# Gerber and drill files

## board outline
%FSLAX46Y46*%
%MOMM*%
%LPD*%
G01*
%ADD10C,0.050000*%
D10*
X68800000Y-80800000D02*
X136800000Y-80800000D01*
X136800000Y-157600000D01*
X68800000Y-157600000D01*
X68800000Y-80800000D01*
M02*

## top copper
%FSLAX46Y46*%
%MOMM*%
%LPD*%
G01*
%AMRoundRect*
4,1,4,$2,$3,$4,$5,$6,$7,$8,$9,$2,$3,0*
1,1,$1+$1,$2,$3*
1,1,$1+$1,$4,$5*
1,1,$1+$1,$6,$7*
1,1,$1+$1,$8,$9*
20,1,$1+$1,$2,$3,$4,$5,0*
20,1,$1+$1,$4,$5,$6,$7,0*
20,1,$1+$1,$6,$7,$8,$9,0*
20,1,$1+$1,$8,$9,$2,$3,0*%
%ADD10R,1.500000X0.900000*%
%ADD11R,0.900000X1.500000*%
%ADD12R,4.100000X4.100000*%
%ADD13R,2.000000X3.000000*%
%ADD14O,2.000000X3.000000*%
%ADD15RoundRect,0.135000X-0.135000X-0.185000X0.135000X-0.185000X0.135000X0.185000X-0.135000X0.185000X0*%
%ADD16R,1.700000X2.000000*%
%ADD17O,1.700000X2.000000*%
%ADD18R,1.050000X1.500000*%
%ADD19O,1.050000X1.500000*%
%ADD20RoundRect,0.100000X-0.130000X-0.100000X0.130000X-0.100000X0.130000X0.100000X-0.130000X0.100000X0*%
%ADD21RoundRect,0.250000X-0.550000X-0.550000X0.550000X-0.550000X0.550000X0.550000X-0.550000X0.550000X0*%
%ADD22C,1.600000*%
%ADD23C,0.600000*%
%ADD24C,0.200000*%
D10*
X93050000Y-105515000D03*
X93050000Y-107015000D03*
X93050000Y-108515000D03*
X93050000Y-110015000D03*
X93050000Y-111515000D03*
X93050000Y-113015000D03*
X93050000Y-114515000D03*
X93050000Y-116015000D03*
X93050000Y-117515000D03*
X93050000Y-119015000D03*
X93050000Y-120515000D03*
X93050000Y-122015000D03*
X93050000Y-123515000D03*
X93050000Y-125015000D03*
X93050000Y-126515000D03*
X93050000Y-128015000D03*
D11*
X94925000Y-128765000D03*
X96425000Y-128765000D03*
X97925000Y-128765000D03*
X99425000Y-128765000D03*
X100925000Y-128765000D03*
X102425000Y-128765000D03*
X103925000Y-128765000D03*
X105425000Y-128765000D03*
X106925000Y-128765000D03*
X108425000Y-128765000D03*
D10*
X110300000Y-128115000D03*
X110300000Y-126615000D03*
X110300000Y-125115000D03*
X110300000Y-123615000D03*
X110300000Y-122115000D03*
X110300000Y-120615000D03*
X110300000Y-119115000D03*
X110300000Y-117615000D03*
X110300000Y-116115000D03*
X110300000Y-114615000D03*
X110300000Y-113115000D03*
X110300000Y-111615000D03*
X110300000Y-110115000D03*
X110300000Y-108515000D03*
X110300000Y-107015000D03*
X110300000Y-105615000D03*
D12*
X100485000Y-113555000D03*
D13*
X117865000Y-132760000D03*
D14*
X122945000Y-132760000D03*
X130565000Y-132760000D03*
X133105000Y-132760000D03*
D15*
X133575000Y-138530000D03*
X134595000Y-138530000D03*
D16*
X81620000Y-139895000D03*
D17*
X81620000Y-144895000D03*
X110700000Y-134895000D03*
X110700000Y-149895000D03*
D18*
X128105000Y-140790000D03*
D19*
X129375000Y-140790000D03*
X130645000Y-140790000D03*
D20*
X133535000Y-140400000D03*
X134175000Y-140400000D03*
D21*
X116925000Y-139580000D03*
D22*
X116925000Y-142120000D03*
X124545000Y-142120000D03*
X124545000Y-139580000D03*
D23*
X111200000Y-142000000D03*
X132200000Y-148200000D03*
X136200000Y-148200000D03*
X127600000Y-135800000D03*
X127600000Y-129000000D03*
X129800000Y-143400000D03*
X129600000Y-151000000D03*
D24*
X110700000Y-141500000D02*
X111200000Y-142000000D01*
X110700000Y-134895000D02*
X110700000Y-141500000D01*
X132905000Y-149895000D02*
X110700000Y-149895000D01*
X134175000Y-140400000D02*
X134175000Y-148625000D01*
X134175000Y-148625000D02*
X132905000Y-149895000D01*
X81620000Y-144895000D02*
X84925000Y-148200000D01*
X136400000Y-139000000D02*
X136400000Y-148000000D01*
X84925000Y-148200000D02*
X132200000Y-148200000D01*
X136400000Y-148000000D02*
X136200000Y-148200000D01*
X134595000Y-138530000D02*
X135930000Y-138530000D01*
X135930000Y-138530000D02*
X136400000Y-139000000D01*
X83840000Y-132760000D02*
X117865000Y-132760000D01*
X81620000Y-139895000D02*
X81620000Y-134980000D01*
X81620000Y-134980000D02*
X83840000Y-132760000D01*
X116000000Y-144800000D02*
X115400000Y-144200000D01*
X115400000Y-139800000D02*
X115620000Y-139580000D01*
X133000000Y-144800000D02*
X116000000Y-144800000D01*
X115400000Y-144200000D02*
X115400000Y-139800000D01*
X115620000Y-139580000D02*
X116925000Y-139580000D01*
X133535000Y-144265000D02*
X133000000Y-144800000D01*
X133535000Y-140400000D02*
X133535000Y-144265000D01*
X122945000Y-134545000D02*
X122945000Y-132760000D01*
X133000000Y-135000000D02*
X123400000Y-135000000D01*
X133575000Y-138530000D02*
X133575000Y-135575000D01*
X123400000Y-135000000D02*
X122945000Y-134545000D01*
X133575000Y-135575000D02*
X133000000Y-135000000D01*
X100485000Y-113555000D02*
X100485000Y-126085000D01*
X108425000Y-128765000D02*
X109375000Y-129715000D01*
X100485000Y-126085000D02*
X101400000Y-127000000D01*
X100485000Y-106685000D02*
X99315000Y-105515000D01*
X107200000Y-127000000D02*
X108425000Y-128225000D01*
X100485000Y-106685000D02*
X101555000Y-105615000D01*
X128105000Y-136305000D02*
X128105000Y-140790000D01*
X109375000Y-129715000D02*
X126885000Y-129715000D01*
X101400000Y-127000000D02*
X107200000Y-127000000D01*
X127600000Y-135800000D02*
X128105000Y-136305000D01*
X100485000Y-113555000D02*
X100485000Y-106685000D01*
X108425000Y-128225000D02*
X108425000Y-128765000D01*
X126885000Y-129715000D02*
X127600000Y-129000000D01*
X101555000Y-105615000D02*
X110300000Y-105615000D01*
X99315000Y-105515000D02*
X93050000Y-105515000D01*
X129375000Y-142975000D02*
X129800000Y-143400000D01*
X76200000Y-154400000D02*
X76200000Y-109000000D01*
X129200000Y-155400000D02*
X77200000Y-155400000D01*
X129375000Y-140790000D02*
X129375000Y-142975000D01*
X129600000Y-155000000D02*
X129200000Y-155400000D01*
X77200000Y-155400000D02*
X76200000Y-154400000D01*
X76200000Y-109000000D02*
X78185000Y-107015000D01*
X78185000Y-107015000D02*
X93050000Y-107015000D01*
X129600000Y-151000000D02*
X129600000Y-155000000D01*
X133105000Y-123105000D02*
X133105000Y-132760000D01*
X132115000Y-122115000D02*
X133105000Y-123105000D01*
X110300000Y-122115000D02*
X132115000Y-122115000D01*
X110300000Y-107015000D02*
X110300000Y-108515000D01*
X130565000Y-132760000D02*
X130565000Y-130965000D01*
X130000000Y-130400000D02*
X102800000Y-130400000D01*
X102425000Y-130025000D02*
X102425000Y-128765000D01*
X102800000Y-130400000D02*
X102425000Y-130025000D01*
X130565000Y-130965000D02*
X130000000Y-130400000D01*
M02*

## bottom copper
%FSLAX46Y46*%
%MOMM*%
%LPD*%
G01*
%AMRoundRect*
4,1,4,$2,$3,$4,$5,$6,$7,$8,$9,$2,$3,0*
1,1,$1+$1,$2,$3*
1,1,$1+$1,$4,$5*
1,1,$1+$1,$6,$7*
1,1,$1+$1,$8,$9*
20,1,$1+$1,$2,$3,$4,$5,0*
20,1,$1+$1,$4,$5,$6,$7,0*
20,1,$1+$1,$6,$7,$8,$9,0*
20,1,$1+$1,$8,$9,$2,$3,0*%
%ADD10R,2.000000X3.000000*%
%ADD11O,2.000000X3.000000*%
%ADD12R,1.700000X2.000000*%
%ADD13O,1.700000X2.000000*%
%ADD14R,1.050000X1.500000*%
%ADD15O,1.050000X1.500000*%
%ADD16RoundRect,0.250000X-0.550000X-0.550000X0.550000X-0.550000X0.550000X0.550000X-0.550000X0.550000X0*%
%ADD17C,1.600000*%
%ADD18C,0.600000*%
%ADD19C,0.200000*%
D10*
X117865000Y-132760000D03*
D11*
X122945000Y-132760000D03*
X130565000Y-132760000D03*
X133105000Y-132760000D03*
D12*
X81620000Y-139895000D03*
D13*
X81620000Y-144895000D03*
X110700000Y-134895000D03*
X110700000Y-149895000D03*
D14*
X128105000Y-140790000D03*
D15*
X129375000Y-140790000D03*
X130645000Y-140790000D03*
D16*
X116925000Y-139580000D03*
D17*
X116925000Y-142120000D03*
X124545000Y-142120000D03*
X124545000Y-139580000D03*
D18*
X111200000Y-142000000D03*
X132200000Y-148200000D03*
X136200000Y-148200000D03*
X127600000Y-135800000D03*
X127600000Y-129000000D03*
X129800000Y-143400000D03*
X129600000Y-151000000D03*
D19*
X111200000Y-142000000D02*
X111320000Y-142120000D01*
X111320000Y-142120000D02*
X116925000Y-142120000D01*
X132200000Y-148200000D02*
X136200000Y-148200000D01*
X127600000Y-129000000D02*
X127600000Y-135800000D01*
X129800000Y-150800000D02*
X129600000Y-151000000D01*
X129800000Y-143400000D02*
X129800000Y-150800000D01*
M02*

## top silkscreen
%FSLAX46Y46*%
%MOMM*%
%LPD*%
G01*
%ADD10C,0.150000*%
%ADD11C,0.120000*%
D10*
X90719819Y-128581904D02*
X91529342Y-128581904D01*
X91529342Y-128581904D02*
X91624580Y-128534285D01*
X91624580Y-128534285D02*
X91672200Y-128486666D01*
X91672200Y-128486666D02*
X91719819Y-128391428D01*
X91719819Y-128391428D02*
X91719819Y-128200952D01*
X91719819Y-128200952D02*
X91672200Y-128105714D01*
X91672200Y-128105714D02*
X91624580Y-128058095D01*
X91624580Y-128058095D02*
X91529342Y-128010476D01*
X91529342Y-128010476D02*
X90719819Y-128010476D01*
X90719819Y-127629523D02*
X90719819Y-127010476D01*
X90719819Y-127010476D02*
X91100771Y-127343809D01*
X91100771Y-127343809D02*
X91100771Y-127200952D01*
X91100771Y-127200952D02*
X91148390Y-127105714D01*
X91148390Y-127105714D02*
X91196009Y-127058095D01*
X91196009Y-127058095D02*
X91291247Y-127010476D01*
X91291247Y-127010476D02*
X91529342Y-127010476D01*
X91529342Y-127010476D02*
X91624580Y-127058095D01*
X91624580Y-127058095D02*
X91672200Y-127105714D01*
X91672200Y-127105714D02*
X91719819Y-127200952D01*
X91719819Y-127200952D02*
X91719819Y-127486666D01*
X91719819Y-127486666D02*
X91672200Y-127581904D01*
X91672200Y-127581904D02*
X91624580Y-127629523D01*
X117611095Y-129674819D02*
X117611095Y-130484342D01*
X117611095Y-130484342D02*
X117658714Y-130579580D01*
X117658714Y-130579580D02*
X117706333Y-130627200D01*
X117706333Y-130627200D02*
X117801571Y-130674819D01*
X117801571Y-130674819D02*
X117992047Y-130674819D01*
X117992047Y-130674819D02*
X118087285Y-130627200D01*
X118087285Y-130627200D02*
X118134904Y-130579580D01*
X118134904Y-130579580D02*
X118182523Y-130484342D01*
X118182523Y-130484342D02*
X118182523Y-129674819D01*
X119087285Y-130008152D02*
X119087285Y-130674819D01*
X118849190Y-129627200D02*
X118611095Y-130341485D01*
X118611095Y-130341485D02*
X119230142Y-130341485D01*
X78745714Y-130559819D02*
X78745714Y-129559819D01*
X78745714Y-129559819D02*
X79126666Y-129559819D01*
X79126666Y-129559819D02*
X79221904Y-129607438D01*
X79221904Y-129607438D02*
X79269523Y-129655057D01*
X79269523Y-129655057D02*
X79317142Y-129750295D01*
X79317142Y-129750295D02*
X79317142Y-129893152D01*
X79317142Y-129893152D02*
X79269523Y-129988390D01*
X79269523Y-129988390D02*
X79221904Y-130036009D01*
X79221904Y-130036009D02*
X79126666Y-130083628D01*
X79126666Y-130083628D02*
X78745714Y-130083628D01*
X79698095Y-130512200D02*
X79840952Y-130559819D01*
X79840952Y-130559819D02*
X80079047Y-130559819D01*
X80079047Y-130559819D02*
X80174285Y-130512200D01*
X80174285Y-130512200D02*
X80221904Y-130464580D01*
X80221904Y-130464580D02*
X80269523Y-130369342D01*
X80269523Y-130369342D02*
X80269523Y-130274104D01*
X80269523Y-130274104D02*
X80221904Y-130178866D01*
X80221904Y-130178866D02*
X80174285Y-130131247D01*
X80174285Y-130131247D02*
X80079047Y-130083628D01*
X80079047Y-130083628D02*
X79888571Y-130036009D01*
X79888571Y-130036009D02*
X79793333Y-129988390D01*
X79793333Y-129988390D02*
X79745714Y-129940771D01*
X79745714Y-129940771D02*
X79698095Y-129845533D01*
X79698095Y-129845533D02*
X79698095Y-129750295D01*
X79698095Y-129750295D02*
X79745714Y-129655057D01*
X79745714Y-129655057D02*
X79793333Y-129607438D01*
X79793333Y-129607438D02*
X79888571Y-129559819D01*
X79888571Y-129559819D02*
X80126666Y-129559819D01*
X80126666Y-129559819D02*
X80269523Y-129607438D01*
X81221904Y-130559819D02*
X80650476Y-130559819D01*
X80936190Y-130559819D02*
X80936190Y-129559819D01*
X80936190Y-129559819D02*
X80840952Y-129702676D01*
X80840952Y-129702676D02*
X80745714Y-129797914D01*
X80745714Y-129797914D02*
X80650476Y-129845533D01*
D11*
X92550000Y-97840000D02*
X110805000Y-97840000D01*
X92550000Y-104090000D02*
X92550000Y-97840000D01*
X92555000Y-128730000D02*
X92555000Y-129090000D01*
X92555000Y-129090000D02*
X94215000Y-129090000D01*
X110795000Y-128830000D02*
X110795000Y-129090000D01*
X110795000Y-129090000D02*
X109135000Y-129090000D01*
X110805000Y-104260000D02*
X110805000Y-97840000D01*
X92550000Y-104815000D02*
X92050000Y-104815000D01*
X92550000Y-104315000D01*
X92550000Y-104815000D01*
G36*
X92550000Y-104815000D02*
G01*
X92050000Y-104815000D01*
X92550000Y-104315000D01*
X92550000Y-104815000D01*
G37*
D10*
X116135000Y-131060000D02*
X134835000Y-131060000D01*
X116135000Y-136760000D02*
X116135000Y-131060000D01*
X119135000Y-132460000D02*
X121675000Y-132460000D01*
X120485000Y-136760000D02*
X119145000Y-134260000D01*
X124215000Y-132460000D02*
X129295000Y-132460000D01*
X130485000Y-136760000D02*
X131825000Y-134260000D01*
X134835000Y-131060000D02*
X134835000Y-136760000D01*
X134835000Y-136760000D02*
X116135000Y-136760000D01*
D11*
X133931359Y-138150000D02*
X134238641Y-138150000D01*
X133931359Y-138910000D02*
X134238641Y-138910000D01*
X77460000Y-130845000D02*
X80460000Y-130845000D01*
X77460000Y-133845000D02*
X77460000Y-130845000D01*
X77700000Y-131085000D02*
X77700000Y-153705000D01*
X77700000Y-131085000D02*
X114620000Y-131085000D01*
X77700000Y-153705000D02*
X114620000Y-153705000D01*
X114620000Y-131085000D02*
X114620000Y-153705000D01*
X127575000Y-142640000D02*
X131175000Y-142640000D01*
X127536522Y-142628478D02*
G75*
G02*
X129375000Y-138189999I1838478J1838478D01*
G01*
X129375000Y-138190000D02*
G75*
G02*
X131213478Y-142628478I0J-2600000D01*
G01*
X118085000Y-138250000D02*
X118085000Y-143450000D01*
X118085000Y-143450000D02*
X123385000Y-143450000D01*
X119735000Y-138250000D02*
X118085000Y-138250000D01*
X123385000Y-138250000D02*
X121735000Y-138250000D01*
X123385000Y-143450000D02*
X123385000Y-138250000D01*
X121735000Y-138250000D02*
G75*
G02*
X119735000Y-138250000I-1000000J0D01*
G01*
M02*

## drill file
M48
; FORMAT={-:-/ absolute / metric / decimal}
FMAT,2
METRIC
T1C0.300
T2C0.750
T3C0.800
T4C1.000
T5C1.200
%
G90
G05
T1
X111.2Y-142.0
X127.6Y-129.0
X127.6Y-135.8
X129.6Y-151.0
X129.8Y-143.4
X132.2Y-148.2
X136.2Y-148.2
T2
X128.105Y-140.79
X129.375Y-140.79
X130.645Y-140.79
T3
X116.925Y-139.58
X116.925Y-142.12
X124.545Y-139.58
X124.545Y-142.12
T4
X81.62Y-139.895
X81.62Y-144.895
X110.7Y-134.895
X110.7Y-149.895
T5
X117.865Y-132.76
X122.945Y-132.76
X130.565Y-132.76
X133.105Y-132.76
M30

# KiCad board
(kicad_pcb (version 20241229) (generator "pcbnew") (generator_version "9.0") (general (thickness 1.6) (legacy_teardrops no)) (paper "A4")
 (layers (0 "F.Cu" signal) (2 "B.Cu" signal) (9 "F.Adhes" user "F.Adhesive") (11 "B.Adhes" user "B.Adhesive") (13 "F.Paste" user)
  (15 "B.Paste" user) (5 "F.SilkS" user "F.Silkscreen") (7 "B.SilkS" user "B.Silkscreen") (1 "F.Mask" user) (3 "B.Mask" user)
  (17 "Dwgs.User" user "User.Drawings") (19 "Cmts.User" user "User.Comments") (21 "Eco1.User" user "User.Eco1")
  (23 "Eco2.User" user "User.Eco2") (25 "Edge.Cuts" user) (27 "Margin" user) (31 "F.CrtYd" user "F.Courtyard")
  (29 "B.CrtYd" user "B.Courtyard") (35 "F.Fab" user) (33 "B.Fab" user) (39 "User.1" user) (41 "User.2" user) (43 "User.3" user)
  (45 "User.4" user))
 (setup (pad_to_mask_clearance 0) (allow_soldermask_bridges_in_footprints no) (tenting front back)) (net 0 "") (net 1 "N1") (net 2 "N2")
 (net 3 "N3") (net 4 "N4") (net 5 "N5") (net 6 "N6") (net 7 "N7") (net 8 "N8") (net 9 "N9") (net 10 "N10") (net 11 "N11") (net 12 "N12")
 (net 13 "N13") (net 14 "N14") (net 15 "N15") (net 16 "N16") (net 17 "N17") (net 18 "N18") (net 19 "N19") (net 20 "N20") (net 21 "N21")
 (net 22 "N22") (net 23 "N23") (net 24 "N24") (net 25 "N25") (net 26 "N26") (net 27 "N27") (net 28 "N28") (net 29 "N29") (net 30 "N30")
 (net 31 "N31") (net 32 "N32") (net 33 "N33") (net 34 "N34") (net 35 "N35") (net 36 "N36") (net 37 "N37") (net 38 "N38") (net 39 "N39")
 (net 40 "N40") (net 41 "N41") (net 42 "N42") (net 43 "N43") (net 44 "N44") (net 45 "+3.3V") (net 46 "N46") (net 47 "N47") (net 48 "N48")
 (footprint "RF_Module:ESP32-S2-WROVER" (layer "F.Cu") (at 101.675 117.29)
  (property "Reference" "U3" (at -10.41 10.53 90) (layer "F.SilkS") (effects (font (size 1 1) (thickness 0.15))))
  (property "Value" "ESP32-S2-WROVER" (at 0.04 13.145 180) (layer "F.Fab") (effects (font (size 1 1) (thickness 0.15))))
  (fp_line (start -9.125 -19.45) (end 9.13 -19.45) (stroke (width 0.12) (type solid)) (layer "F.SilkS"))
  (fp_line (start -9.125 -13.2) (end -9.125 -19.45) (stroke (width 0.12) (type solid)) (layer "F.SilkS"))
  (fp_line (start -9.12 11.44) (end -9.12 11.8) (stroke (width 0.12) (type solid)) (layer "F.SilkS"))
  (fp_line (start -9.12 11.8) (end -7.46 11.8) (stroke (width 0.12) (type solid)) (layer "F.SilkS"))
  (fp_line (start 9.12 11.54) (end 9.12 11.8) (stroke (width 0.12) (type solid)) (layer "F.SilkS"))
  (fp_line (start 9.12 11.8) (end 7.46 11.8) (stroke (width 0.12) (type solid)) (layer "F.SilkS"))
  (fp_line (start 9.13 -13.03) (end 9.13 -19.45) (stroke (width 0.12) (type solid)) (layer "F.SilkS"))
  (fp_poly
   (pts (xy -9.125 -12.475) (xy -9.625 -12.475) (xy -9.125 -12.975) (xy -9.125 -12.475)) (stroke (width 0.12) (type solid)) (fill yes)
   (layer "F.SilkS"))
  (pad "" smd roundrect (at -2.52 -5.065) (size 1.07 1.07) (layers "F.Paste") (roundrect_rratio 0.233645))
  (pad "" smd roundrect (at -2.52 -3.735) (size 1.07 1.07) (layers "F.Paste") (roundrect_rratio 0.233645))
  (pad "" smd roundrect (at -2.52 -2.405) (size 1.07 1.07) (layers "F.Paste") (roundrect_rratio 0.233645))
  (pad "" smd roundrect (at -1.19 -5.065) (size 1.07 1.07) (layers "F.Paste") (roundrect_rratio 0.233645))
  (pad "" smd roundrect (at -1.19 -3.735) (size 1.07 1.07) (layers "F.Paste") (roundrect_rratio 0.233645))
  (pad "" smd roundrect (at -1.19 -2.405) (size 1.07 1.07) (layers "F.Paste") (roundrect_rratio 0.233645))
  (pad "" smd roundrect (at 0.14 -5.065) (size 1.07 1.07) (layers "F.Paste") (roundrect_rratio 0.233645))
  (pad "" smd roundrect (at 0.14 -3.735) (size 1.07 1.07) (layers "F.Paste") (roundrect_rratio 0.233645))
  (pad "" smd roundrect (at 0.14 -2.405) (size 1.07 1.07) (layers "F.Paste") (roundrect_rratio 0.233645))
  (pad "1" smd rect (at -8.625 -11.775) (size 1.5 0.9) (layers "F.Cu" "F.Mask" "F.Paste") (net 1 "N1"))
  (pad "2" smd rect (at -8.625 -10.275) (size 1.5 0.9) (layers "F.Cu" "F.Mask" "F.Paste") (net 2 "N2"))
  (pad "3" smd rect (at -8.625 -8.775) (size 1.5 0.9) (layers "F.Cu" "F.Mask" "F.Paste") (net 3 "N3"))
  (pad "4" smd rect (at -8.625 -7.275) (size 1.5 0.9) (layers "F.Cu" "F.Mask" "F.Paste") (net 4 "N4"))
  (pad "5" smd rect (at -8.625 -5.775) (size 1.5 0.9) (layers "F.Cu" "F.Mask" "F.Paste") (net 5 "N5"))
  (pad "6" smd rect (at -8.625 -4.275) (size 1.5 0.9) (layers "F.Cu" "F.Mask" "F.Paste") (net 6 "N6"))
  (pad "7" smd rect (at -8.625 -2.775) (size 1.5 0.9) (layers "F.Cu" "F.Mask" "F.Paste") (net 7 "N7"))
  (pad "8" smd rect (at -8.625 -1.275) (size 1.5 0.9) (layers "F.Cu" "F.Mask" "F.Paste") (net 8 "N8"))
  (pad "9" smd rect (at -8.625 0.225) (size 1.5 0.9) (layers "F.Cu" "F.Mask" "F.Paste") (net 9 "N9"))
  (pad "10" smd rect (at -8.625 1.725) (size 1.5 0.9) (layers "F.Cu" "F.Mask" "F.Paste") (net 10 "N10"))
  (pad "11" smd rect (at -8.625 3.225) (size 1.5 0.9) (layers "F.Cu" "F.Mask" "F.Paste") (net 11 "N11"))
  (pad "12" smd rect (at -8.625 4.725) (size 1.5 0.9) (layers "F.Cu" "F.Mask" "F.Paste") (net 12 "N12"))
  (pad "13" smd rect (at -8.625 6.225) (size 1.5 0.9) (layers "F.Cu" "F.Mask" "F.Paste") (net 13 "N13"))
  (pad "14" smd rect (at -8.625 7.725) (size 1.5 0.9) (layers "F.Cu" "F.Mask" "F.Paste") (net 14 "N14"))
  (pad "15" smd rect (at -8.625 9.225 180) (size 1.5 0.9) (layers "F.Cu" "F.Mask" "F.Paste") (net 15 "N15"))
  (pad "16" smd rect (at -8.625 10.725 180) (size 1.5 0.9) (layers "F.Cu" "F.Mask" "F.Paste") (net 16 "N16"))
  (pad "17" smd rect (at -6.75 11.475) (size 0.9 1.5) (layers "F.Cu" "F.Mask" "F.Paste") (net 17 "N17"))
  (pad "18" smd rect (at -5.25 11.475) (size 0.9 1.5) (layers "F.Cu" "F.Mask" "F.Paste") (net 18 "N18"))
  (pad "19" smd rect (at -3.75 11.475) (size 0.9 1.5) (layers "F.Cu" "F.Mask" "F.Paste") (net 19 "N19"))
  (pad "20" smd rect (at -2.25 11.475) (size 0.9 1.5) (layers "F.Cu" "F.Mask" "F.Paste") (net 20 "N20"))
  (pad "21" smd rect (at -0.75 11.475) (size 0.9 1.5) (layers "F.Cu" "F.Mask" "F.Paste") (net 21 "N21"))
  (pad "22" smd rect (at 0.75 11.475) (size 0.9 1.5) (layers "F.Cu" "F.Mask" "F.Paste") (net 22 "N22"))
  (pad "23" smd rect (at 2.25 11.475) (size 0.9 1.5) (layers "F.Cu" "F.Mask" "F.Paste") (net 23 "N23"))
  (pad "24" smd rect (at 3.75 11.475) (size 0.9 1.5) (layers "F.Cu" "F.Mask" "F.Paste") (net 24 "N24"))
  (pad "25" smd rect (at 5.25 11.475) (size 0.9 1.5) (layers "F.Cu" "F.Mask" "F.Paste") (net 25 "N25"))
  (pad "26" smd rect (at 6.75 11.475) (size 0.9 1.5) (layers "F.Cu" "F.Mask" "F.Paste") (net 1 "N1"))
  (pad "27" smd rect (at 8.625 10.825) (size 1.5 0.9) (layers "F.Cu" "F.Mask" "F.Paste") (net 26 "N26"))
  (pad "28" smd rect (at 8.625 9.325) (size 1.5 0.9) (layers "F.Cu" "F.Mask" "F.Paste") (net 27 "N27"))
  (pad "29" smd rect (at 8.625 7.825) (size 1.5 0.9) (layers "F.Cu" "F.Mask" "F.Paste") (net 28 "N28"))
  (pad "30" smd rect (at 8.625 6.325) (size 1.5 0.9) (layers "F.Cu" "F.Mask" "F.Paste") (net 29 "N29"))
  (pad "31" smd rect (at 8.625 4.825) (size 1.5 0.9) (layers "F.Cu" "F.Mask" "F.Paste") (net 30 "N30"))
  (pad "32" smd rect (at 8.625 3.325) (size 1.5 0.9) (layers "F.Cu" "F.Mask" "F.Paste") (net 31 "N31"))
  (pad "33" smd rect (at 8.625 1.825) (size 1.5 0.9) (layers "F.Cu" "F.Mask" "F.Paste") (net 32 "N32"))
  (pad "34" smd rect (at 8.625 0.325) (size 1.5 0.9) (layers "F.Cu" "F.Mask" "F.Paste") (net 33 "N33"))
  (pad "35" smd rect (at 8.625 -1.175) (size 1.5 0.9) (layers "F.Cu" "F.Mask" "F.Paste") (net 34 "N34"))
  (pad "36" smd rect (at 8.625 -2.675) (size 1.5 0.9) (layers "F.Cu" "F.Mask" "F.Paste") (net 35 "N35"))
  (pad "37" smd rect (at 8.625 -4.175) (size 1.5 0.9) (layers "F.Cu" "F.Mask" "F.Paste") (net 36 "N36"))
  (pad "38" smd rect (at 8.625 -5.675) (size 1.5 0.9) (layers "F.Cu" "F.Mask" "F.Paste") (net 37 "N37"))
  (pad "39" smd rect (at 8.625 -7.175) (size 1.5 0.9) (layers "F.Cu" "F.Mask" "F.Paste") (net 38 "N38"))
  (pad "40" smd rect (at 8.625 -8.775) (size 1.5 0.9) (layers "F.Cu" "F.Mask" "F.Paste") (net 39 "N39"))
  (pad "41" smd rect (at 8.625 -10.275) (size 1.5 0.9) (layers "F.Cu" "F.Mask" "F.Paste") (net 39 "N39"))
  (pad "42" smd rect (at 8.625 -11.675) (size 1.5 0.9) (layers "F.Cu" "F.Mask" "F.Paste") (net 1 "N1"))
  (pad "43" smd rect (at -1.19 -3.735) (size 4.1 4.1) (layers "F.Cu" "F.Mask") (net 1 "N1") (zone_connect 2))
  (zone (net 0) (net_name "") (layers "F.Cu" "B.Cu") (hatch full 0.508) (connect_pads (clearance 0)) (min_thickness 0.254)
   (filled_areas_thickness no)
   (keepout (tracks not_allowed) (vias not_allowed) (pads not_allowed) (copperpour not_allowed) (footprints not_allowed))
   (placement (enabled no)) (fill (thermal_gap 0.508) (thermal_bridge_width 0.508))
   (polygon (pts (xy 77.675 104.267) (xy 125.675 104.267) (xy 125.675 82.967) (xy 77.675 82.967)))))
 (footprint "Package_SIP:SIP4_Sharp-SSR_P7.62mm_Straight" (layer "F.Cu") (at 117.865 132.76)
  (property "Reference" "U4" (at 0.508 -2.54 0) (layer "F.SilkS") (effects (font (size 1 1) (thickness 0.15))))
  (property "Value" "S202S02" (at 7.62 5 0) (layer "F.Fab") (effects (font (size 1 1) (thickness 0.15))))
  (fp_line (start -1.73 -1.7) (end 16.97 -1.7) (stroke (width 0.15) (type solid)) (layer "F.SilkS"))
  (fp_line (start -1.73 4) (end -1.73 -1.7) (stroke (width 0.15) (type solid)) (layer "F.SilkS"))
  (fp_line (start 1.27 -0.3) (end 3.81 -0.3) (stroke (width 0.15) (type solid)) (layer "F.SilkS"))
  (fp_line (start 2.62 4) (end 1.28 1.5) (stroke (width 0.15) (type solid)) (layer "F.SilkS"))
  (fp_line (start 6.35 -0.3) (end 11.43 -0.3) (stroke (width 0.15) (type solid)) (layer "F.SilkS"))
  (fp_line (start 12.62 4) (end 13.96 1.5) (stroke (width 0.15) (type solid)) (layer "F.SilkS"))
  (fp_line (start 16.97 -1.7) (end 16.97 4) (stroke (width 0.15) (type solid)) (layer "F.SilkS"))
  (fp_line (start 16.97 4) (end -1.73 4) (stroke (width 0.15) (type solid)) (layer "F.SilkS"))
  (pad "1" thru_hole rect (at 0 0) (size 2 3) (drill 1.2) (layers "*.Cu" "*.Mask") (remove_unused_layers no) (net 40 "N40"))
  (pad "2" thru_hole oval (at 5.08 0) (size 2 3) (drill 1.2) (layers "*.Cu" "*.Mask") (remove_unused_layers no) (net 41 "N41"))
  (pad "3" thru_hole oval (at 12.7 0) (size 2 3) (drill 1.2) (layers "*.Cu" "*.Mask") (remove_unused_layers no) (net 22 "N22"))
  (pad "4" thru_hole oval (at 15.24 0) (size 2 3) (drill 1.2) (layers "*.Cu" "*.Mask") (remove_unused_layers no) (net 30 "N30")))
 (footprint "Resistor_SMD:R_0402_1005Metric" (layer "F.Cu") (at 134.085 138.53)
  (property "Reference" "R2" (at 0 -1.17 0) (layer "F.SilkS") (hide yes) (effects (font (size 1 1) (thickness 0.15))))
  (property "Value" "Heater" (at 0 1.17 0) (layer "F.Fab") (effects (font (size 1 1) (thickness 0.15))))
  (fp_line (start -0.153641 -0.38) (end 0.153641 -0.38) (stroke (width 0.12) (type solid)) (layer "F.SilkS"))
  (fp_line (start -0.153641 0.38) (end 0.153641 0.38) (stroke (width 0.12) (type solid)) (layer "F.SilkS"))
  (pad "1" smd roundrect (at -0.51 0) (size 0.54 0.64) (layers "F.Cu" "F.Mask" "F.Paste") (roundrect_rratio 0.25) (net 41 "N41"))
  (pad "2" smd roundrect (at 0.51 0) (size 0.54 0.64) (layers "F.Cu" "F.Mask" "F.Paste") (roundrect_rratio 0.25) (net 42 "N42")))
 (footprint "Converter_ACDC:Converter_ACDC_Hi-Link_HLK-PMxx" (layer "F.Cu") (at 81.62 139.895)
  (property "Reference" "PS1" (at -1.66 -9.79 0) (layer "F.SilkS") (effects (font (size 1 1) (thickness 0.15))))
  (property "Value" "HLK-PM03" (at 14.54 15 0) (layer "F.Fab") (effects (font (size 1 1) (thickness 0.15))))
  (fp_line (start -4.16 -9.05) (end -1.16 -9.05) (stroke (width 0.12) (type solid)) (layer "F.SilkS"))
  (fp_line (start -4.16 -6.05) (end -4.16 -9.05) (stroke (width 0.12) (type solid)) (layer "F.SilkS"))
  (fp_line (start -3.92 -8.81) (end -3.92 13.81) (stroke (width 0.12) (type solid)) (layer "F.SilkS"))
  (fp_line (start -3.92 -8.81) (end 33 -8.81) (stroke (width 0.12) (type solid)) (layer "F.SilkS"))
  (fp_line (start -3.92 13.81) (end 33 13.81) (stroke (width 0.12) (type solid)) (layer "F.SilkS"))
  (fp_line (start 33 -8.81) (end 33 13.81) (stroke (width 0.12) (type solid)) (layer "F.SilkS"))
  (pad "1" thru_hole rect (at 0 0) (size 1.7 2) (drill 1) (layers "*.Cu" "*.Mask") (remove_unused_layers no) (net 40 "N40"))
  (pad "2" thru_hole oval (at 0 5) (size 1.7 2) (drill 1) (layers "*.Cu" "*.Mask") (remove_unused_layers no) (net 42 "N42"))
  (pad "3" thru_hole oval (at 29.08 -5) (size 1.7 2) (drill 1) (layers "*.Cu" "*.Mask") (remove_unused_layers no) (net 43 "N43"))
  (pad "4" thru_hole oval (at 29.08 10) (size 1.7 2) (drill 1) (layers "*.Cu" "*.Mask") (remove_unused_layers no) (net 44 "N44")))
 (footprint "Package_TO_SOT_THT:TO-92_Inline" (layer "F.Cu") (at 128.105 140.79)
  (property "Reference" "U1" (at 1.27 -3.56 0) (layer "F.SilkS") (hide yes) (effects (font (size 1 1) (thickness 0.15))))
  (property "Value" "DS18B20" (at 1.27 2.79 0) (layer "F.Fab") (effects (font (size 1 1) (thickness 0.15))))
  (fp_line (start -0.53 1.85) (end 3.07 1.85) (stroke (width 0.12) (type solid)) (layer "F.SilkS"))
  (fp_arc (start -0.568478 1.838478) (mid -1.132087 -0.994977) (end 1.27 -2.6) (stroke (width 0.12) (type solid)) (layer "F.SilkS"))
  (fp_arc (start 1.27 -2.6) (mid 3.672087 -0.994977) (end 3.108478 1.838478) (stroke (width 0.12) (type solid)) (layer "F.SilkS"))
  (pad "1" thru_hole rect (at 0 0) (size 1.05 1.5) (drill 0.75) (layers "*.Cu" "*.Mask") (remove_unused_layers no) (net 1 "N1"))
  (pad "2" thru_hole oval (at 1.27 0) (size 1.05 1.5) (drill 0.75) (layers "*.Cu" "*.Mask") (remove_unused_layers no) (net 2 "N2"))
  (pad "3" thru_hole oval (at 2.54 0) (size 1.05 1.5) (drill 0.75) (layers "*.Cu" "*.Mask") (remove_unused_layers no) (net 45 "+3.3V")))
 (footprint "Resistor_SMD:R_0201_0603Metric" (layer "F.Cu") (at 133.855 140.4)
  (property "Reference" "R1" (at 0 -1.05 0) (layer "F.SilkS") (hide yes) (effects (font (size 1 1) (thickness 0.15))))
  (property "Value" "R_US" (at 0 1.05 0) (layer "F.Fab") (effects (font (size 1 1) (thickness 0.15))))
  (pad "" smd roundrect (at -0.345 0) (size 0.318 0.36) (layers "F.Paste") (roundrect_rratio 0.25))
  (pad "" smd roundrect (at 0.345 0) (size 0.318 0.36) (layers "F.Paste") (roundrect_rratio 0.25))
  (pad "1" smd roundrect (at -0.32 0) (size 0.46 0.4) (layers "F.Cu" "F.Mask") (roundrect_rratio 0.25) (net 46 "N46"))
  (pad "2" smd roundrect (at 0.32 0) (size 0.46 0.4) (layers "F.Cu" "F.Mask") (roundrect_rratio 0.25) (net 44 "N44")))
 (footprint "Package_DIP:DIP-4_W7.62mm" (layer "F.Cu") (at 116.925 139.58)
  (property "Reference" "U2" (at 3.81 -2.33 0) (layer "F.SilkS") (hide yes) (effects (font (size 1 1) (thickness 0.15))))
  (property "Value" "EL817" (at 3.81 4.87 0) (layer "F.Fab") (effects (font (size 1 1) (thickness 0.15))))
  (fp_line (start 1.16 -1.33) (end 1.16 3.87) (stroke (width 0.12) (type solid)) (layer "F.SilkS"))
  (fp_line (start 1.16 3.87) (end 6.46 3.87) (stroke (width 0.12) (type solid)) (layer "F.SilkS"))
  (fp_line (start 2.81 -1.33) (end 1.16 -1.33) (stroke (width 0.12) (type solid)) (layer "F.SilkS"))
  (fp_line (start 6.46 -1.33) (end 4.81 -1.33) (stroke (width 0.12) (type solid)) (layer "F.SilkS"))
  (fp_line (start 6.46 3.87) (end 6.46 -1.33) (stroke (width 0.12) (type solid)) (layer "F.SilkS"))
  (fp_arc (start 4.81 -1.33) (mid 3.81 -0.33) (end 2.81 -1.33) (stroke (width 0.12) (type solid)) (layer "F.SilkS"))
  (pad "1" thru_hole roundrect (at 0 0) (size 1.6 1.6) (drill 0.8) (layers "*.Cu" "*.Mask") (remove_unused_layers no)
   (roundrect_rratio 0.15625) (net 46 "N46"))
  (pad "2" thru_hole circle (at 0 2.54) (size 1.6 1.6) (drill 0.8) (layers "*.Cu" "*.Mask") (remove_unused_layers no) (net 43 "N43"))
  (pad "3" thru_hole circle (at 7.62 2.54) (size 1.6 1.6) (drill 0.8) (layers "*.Cu" "*.Mask") (remove_unused_layers no) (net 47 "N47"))
  (pad "4" thru_hole circle (at 7.62 0) (size 1.6 1.6) (drill 0.8) (layers "*.Cu" "*.Mask") (remove_unused_layers no) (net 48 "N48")))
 (gr_rect (start 68.8 80.8) (end 136.8 157.6) (stroke (width 0.05) (type default)) (fill no) (layer "Edge.Cuts"))
 (segment (start 110.7 141.5) (end 111.2 142) (width 0.2) (layer "F.Cu") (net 43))
 (segment (start 110.7 134.895) (end 110.7 141.5) (width 0.2) (layer "F.Cu") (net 43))
 (via (at 111.2 142) (size 0.6) (drill 0.3) (layers "F.Cu" "B.Cu") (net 43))
 (segment (start 111.2 142) (end 111.32 142.12) (width 0.2) (layer "B.Cu") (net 43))
 (segment (start 111.32 142.12) (end 116.925 142.12) (width 0.2) (layer "B.Cu") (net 43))
 (segment (start 132.905 149.895) (end 110.7 149.895) (width 0.2) (layer "F.Cu") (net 44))
 (segment (start 134.175 140.4) (end 134.175 148.625) (width 0.2) (layer "F.Cu") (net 44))
 (segment (start 134.175 148.625) (end 132.905 149.895) (width 0.2) (layer "F.Cu") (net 44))
 (segment (start 81.62 144.895) (end 84.925 148.2) (width 0.2) (layer "F.Cu") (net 42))
 (segment (start 136.4 139) (end 136.4 148) (width 0.2) (layer "F.Cu") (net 42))
 (segment (start 84.925 148.2) (end 132.2 148.2) (width 0.2) (layer "F.Cu") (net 42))
 (segment (start 136.4 148) (end 136.2 148.2) (width 0.2) (layer "F.Cu") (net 42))
 (segment (start 134.595 138.53) (end 135.93 138.53) (width 0.2) (layer "F.Cu") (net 42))
 (segment (start 135.93 138.53) (end 136.4 139) (width 0.2) (layer "F.Cu") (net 42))
 (via (at 132.2 148.2) (size 0.6) (drill 0.3) (layers "F.Cu" "B.Cu") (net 42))
 (via (at 136.2 148.2) (size 0.6) (drill 0.3) (layers "F.Cu" "B.Cu") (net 42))
 (segment (start 132.2 148.2) (end 136.2 148.2) (width 0.2) (layer "B.Cu") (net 42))
 (segment (start 83.84 132.76) (end 117.865 132.76) (width 0.2) (layer "F.Cu") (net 40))
 (segment (start 81.62 139.895) (end 81.62 134.98) (width 0.2) (layer "F.Cu") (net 40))
 (segment (start 81.62 134.98) (end 83.84 132.76) (width 0.2) (layer "F.Cu") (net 40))
 (segment (start 116 144.8) (end 115.4 144.2) (width 0.2) (layer "F.Cu") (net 46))
 (segment (start 115.4 139.8) (end 115.62 139.58) (width 0.2) (layer "F.Cu") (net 46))
 (segment (start 133 144.8) (end 116 144.8) (width 0.2) (layer "F.Cu") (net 46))
 (segment (start 115.4 144.2) (end 115.4 139.8) (width 0.2) (layer "F.Cu") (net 46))
 (segment (start 115.62 139.58) (end 116.925 139.58) (width 0.2) (layer "F.Cu") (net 46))
 (segment (start 133.535 144.265) (end 133 144.8) (width 0.2) (layer "F.Cu") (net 46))
 (segment (start 133.535 140.4) (end 133.535 144.265) (width 0.2) (layer "F.Cu") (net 46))
 (segment (start 122.945 134.545) (end 122.945 132.76) (width 0.2) (layer "F.Cu") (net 41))
 (segment (start 133 135) (end 123.4 135) (width 0.2) (layer "F.Cu") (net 41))
 (segment (start 133.575 138.53) (end 133.575 135.575) (width 0.2) (layer "F.Cu") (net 41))
 (segment (start 123.4 135) (end 122.945 134.545) (width 0.2) (layer "F.Cu") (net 41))
 (segment (start 133.575 135.575) (end 133 135) (width 0.2) (layer "F.Cu") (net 41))
 (segment (start 100.485 113.555) (end 100.485 126.085) (width 0.2) (layer "F.Cu") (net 1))
 (segment (start 108.425 128.765) (end 109.375 129.715) (width 0.2) (layer "F.Cu") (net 1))
 (segment (start 100.485 126.085) (end 101.4 127) (width 0.2) (layer "F.Cu") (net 1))
 (segment (start 100.485 106.685) (end 99.315 105.515) (width 0.2) (layer "F.Cu") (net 1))
 (segment (start 107.2 127) (end 108.425 128.225) (width 0.2) (layer "F.Cu") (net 1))
 (segment (start 100.485 106.685) (end 101.555 105.615) (width 0.2) (layer "F.Cu") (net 1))
 (segment (start 128.105 136.305) (end 128.105 140.79) (width 0.2) (layer "F.Cu") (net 1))
 (segment (start 109.375 129.715) (end 126.885 129.715) (width 0.2) (layer "F.Cu") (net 1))
 (segment (start 101.4 127) (end 107.2 127) (width 0.2) (layer "F.Cu") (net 1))
 (segment (start 127.6 135.8) (end 128.105 136.305) (width 0.2) (layer "F.Cu") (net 1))
 (segment (start 100.485 113.555) (end 100.485 106.685) (width 0.2) (layer "F.Cu") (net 1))
 (segment (start 108.425 128.225) (end 108.425 128.765) (width 0.2) (layer "F.Cu") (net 1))
 (segment (start 126.885 129.715) (end 127.6 129) (width 0.2) (layer "F.Cu") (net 1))
 (segment (start 101.555 105.615) (end 110.3 105.615) (width 0.2) (layer "F.Cu") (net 1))
 (segment (start 99.315 105.515) (end 93.05 105.515) (width 0.2) (layer "F.Cu") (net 1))
 (via (at 127.6 135.8) (size 0.6) (drill 0.3) (layers "F.Cu" "B.Cu") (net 1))
 (via (at 127.6 129) (size 0.6) (drill 0.3) (layers "F.Cu" "B.Cu") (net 1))
 (segment (start 127.6 129) (end 127.6 135.8) (width 0.2) (layer "B.Cu") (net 1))
 (segment (start 129.375 142.975) (end 129.8 143.4) (width 0.2) (layer "F.Cu") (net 2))
 (segment (start 76.2 154.4) (end 76.2 109) (width 0.2) (layer "F.Cu") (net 2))
 (segment (start 129.2 155.4) (end 77.2 155.4) (width 0.2) (layer "F.Cu") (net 2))
 (segment (start 129.375 140.79) (end 129.375 142.975) (width 0.2) (layer "F.Cu") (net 2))
 (segment (start 129.6 155) (end 129.2 155.4) (width 0.2) (layer "F.Cu") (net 2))
 (segment (start 77.2 155.4) (end 76.2 154.4) (width 0.2) (layer "F.Cu") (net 2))
 (segment (start 76.2 109) (end 78.185 107.015) (width 0.2) (layer "F.Cu") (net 2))
 (segment (start 78.185 107.015) (end 93.05 107.015) (width 0.2) (layer "F.Cu") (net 2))
 (segment (start 129.6 151) (end 129.6 155) (width 0.2) (layer "F.Cu") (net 2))
 (via (at 129.8 143.4) (size 0.6) (drill 0.3) (layers "F.Cu" "B.Cu") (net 2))
 (via (at 129.6 151) (size 0.6) (drill 0.3) (layers "F.Cu" "B.Cu") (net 2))
 (segment (start 129.8 150.8) (end 129.6 151) (width 0.2) (layer "B.Cu") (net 2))
 (segment (start 129.8 143.4) (end 129.8 150.8) (width 0.2) (layer "B.Cu") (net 2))
 (segment (start 133.105 123.105) (end 133.105 132.76) (width 0.2) (layer "F.Cu") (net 30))
 (segment (start 132.115 122.115) (end 133.105 123.105) (width 0.2) (layer "F.Cu") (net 30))
 (segment (start 110.3 122.115) (end 132.115 122.115) (width 0.2) (layer "F.Cu") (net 30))
 (segment (start 110.3 107.015) (end 110.3 108.515) (width 0.2) (layer "F.Cu") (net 39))
 (segment (start 130.565 132.76) (end 130.565 130.965) (width 0.2) (layer "F.Cu") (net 22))
 (segment (start 130 130.4) (end 102.8 130.4) (width 0.2) (layer "F.Cu") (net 22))
 (segment (start 102.425 130.025) (end 102.425 128.765) (width 0.2) (layer "F.Cu") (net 22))
 (segment (start 102.8 130.4) (end 102.425 130.025) (width 0.2) (layer "F.Cu") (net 22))
 (segment (start 130.565 130.965) (end 130 130.4) (width 0.2) (layer "F.Cu") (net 22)))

